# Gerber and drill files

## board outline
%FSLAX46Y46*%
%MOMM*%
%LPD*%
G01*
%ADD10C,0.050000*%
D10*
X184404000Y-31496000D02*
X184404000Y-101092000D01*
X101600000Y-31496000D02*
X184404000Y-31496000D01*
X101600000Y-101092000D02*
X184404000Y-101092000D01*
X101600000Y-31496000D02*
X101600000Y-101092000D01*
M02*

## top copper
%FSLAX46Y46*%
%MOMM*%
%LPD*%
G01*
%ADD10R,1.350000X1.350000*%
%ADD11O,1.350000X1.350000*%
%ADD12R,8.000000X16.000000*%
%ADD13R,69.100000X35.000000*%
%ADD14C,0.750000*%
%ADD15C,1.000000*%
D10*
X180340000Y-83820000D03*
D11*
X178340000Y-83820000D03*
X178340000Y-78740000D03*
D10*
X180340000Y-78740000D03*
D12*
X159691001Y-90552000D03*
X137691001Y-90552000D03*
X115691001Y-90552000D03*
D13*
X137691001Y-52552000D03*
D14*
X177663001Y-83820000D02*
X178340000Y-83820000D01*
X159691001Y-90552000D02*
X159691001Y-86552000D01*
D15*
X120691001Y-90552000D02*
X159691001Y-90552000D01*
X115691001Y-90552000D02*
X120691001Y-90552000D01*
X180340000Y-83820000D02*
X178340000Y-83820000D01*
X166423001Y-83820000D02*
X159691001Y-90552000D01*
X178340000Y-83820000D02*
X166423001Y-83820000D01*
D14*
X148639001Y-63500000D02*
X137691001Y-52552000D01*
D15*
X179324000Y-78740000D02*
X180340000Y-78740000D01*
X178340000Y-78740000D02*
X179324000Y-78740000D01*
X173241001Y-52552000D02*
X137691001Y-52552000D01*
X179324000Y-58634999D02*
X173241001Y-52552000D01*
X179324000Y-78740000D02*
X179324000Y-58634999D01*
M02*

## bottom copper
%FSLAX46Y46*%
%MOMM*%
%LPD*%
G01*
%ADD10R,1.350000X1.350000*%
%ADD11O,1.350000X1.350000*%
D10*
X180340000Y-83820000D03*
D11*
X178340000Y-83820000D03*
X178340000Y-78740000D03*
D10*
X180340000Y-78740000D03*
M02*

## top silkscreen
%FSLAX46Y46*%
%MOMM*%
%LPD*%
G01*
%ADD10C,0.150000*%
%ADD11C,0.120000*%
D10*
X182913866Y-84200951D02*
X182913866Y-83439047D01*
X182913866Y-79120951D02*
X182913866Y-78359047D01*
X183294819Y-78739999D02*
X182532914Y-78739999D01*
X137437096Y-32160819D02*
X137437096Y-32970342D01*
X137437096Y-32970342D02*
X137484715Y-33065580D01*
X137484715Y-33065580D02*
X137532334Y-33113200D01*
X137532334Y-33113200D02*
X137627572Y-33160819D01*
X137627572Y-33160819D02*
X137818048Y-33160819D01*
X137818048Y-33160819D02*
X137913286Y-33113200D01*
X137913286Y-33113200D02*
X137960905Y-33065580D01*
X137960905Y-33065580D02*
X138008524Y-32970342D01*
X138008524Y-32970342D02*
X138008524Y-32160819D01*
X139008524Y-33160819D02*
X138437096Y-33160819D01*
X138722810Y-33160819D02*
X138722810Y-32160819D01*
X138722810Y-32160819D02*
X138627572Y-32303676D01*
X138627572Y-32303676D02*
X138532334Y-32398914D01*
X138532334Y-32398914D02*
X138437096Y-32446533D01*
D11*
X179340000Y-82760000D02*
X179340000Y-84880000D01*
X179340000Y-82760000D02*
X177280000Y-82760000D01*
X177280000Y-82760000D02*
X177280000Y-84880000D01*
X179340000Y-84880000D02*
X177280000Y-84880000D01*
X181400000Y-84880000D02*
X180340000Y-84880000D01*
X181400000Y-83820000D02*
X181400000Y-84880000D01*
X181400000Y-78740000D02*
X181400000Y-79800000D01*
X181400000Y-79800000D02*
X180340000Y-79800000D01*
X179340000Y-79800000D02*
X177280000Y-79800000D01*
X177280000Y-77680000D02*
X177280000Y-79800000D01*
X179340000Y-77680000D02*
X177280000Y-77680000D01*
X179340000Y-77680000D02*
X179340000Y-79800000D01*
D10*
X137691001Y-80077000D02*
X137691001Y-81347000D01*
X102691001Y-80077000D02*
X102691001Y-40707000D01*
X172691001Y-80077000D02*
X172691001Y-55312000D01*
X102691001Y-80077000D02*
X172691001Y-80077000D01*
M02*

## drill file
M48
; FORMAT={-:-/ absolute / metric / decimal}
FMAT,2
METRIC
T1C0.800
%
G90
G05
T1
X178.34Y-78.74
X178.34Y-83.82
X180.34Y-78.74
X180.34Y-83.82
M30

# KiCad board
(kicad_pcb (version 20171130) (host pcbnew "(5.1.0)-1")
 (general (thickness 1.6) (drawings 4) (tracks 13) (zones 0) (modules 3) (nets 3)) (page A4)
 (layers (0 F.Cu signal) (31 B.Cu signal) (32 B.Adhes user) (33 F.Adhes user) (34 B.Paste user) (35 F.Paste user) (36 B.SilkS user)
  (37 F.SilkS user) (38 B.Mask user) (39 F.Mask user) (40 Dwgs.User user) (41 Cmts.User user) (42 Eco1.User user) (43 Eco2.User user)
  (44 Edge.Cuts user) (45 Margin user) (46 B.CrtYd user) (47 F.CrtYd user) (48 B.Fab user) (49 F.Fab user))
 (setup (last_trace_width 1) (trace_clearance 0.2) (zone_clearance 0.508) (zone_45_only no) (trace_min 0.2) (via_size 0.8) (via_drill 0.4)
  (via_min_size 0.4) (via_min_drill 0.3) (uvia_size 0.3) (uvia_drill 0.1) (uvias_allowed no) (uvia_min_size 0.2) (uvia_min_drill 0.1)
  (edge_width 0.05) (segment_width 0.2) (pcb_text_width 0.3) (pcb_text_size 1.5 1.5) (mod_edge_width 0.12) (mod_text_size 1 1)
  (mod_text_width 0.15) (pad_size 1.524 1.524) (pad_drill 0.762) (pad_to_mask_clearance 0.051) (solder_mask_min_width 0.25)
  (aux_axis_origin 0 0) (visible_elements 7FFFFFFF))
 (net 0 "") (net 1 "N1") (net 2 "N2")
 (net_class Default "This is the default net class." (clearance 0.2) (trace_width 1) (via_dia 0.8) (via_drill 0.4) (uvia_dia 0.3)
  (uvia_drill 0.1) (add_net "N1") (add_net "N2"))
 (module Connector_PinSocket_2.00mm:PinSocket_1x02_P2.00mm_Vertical (layer F.Cu) (at 180.34 83.82 270)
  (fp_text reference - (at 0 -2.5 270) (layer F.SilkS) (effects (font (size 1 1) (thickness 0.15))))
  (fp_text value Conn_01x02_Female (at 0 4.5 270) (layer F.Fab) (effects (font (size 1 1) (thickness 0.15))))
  (fp_line (start -1.06 1) (end 1.06 1) (layer F.SilkS) (width 0.12))
  (fp_line (start -1.06 1) (end -1.06 3.06) (layer F.SilkS) (width 0.12))
  (fp_line (start -1.06 3.06) (end 1.06 3.06) (layer F.SilkS) (width 0.12))
  (fp_line (start 1.06 1) (end 1.06 3.06) (layer F.SilkS) (width 0.12))
  (fp_line (start 1.06 -1.06) (end 1.06 0) (layer F.SilkS) (width 0.12))
  (fp_line (start 0 -1.06) (end 1.06 -1.06) (layer F.SilkS) (width 0.12))
  (pad 1 thru_hole rect (at 0 0 270) (size 1.35 1.35) (drill 0.8) (layers *.Cu *.Mask) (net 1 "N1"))
  (pad 2 thru_hole oval (at 0 2 270) (size 1.35 1.35) (drill 0.8) (layers *.Cu *.Mask) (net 1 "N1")))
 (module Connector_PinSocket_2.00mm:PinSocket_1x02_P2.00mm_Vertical (layer F.Cu) (at 180.34 78.74 270)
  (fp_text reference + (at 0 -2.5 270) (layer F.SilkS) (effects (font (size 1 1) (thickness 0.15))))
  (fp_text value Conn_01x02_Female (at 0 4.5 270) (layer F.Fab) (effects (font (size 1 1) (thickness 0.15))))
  (fp_line (start 0 -1.06) (end 1.06 -1.06) (layer F.SilkS) (width 0.12))
  (fp_line (start 1.06 -1.06) (end 1.06 0) (layer F.SilkS) (width 0.12))
  (fp_line (start 1.06 1) (end 1.06 3.06) (layer F.SilkS) (width 0.12))
  (fp_line (start -1.06 3.06) (end 1.06 3.06) (layer F.SilkS) (width 0.12))
  (fp_line (start -1.06 1) (end -1.06 3.06) (layer F.SilkS) (width 0.12))
  (fp_line (start -1.06 1) (end 1.06 1) (layer F.SilkS) (width 0.12))
  (pad 2 thru_hole oval (at 0 2 270) (size 1.35 1.35) (drill 0.8) (layers *.Cu *.Mask) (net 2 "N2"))
  (pad 1 thru_hole rect (at 0 0 270) (size 1.35 1.35) (drill 0.8) (layers *.Cu *.Mask) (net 2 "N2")))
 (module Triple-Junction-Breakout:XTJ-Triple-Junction (layer F.Cu) (at 137.691001 70.552)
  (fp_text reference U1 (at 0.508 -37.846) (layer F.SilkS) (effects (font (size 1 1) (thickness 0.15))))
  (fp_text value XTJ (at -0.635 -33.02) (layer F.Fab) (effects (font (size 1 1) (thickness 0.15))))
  (fp_line (start 0 9.525) (end 0 10.795) (layer F.SilkS) (width 0.15))
  (fp_line (start -35 9.525) (end -35 -29.845) (layer F.SilkS) (width 0.15))
  (fp_line (start 35 9.525) (end 35 -15.24) (layer F.SilkS) (width 0.15))
  (fp_line (start -35 9.525) (end 35 9.525) (layer F.SilkS) (width 0.15))
  (pad 3 smd rect (at 22 20) (size 8 16) (layers F.Cu F.Paste F.Mask) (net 1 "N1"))
  (pad 2 smd rect (at 0 20) (size 8 16) (layers F.Cu F.Paste F.Mask) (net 1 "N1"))
  (pad 1 smd rect (at -22 20) (size 8 16) (layers F.Cu F.Paste F.Mask) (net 1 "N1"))
  (pad 4 smd rect (at 0 -18) (size 69.1 35) (layers F.Cu F.Paste F.Mask) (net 2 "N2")))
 (gr_line (start 184.404 31.496) (end 184.404 101.092) (layer Edge.Cuts) (width 0.05))
 (gr_line (start 101.6 31.496) (end 184.404 31.496) (layer Edge.Cuts) (width 0.05))
 (gr_line (start 101.6 101.092) (end 184.404 101.092) (layer Edge.Cuts) (width 0.05))
 (gr_line (start 101.6 31.496) (end 101.6 101.092) (layer Edge.Cuts) (width 0.05))
 (segment (start 177.663001 83.82) (end 178.34 83.82) (width 0.75) (layer F.Cu) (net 1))
 (segment (start 159.691001 90.552) (end 159.691001 86.552) (width 0.75) (layer F.Cu) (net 1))
 (segment (start 120.691001 90.552) (end 159.691001 90.552) (width 1) (layer F.Cu) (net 1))
 (segment (start 115.691001 90.552) (end 120.691001 90.552) (width 1) (layer F.Cu) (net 1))
 (segment (start 180.34 83.82) (end 178.34 83.82) (width 1) (layer F.Cu) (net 1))
 (segment (start 166.423001 83.82) (end 159.691001 90.552) (width 1) (layer F.Cu) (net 1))
 (segment (start 178.34 83.82) (end 166.423001 83.82) (width 1) (layer F.Cu) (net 1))
 (segment (start 148.639001 63.5) (end 137.691001 52.552) (width 0.75) (layer F.Cu) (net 2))
 (segment (start 179.324 78.74) (end 180.34 78.74) (width 1) (layer F.Cu) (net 2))
 (segment (start 178.34 78.74) (end 179.324 78.74) (width 1) (layer F.Cu) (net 2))
 (segment (start 173.241001 52.552) (end 137.691001 52.552) (width 1) (layer F.Cu) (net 2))
 (segment (start 179.324 58.634999) (end 173.241001 52.552) (width 1) (layer F.Cu) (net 2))
 (segment (start 179.324 78.74) (end 179.324 58.634999) (width 1) (layer F.Cu) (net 2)))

